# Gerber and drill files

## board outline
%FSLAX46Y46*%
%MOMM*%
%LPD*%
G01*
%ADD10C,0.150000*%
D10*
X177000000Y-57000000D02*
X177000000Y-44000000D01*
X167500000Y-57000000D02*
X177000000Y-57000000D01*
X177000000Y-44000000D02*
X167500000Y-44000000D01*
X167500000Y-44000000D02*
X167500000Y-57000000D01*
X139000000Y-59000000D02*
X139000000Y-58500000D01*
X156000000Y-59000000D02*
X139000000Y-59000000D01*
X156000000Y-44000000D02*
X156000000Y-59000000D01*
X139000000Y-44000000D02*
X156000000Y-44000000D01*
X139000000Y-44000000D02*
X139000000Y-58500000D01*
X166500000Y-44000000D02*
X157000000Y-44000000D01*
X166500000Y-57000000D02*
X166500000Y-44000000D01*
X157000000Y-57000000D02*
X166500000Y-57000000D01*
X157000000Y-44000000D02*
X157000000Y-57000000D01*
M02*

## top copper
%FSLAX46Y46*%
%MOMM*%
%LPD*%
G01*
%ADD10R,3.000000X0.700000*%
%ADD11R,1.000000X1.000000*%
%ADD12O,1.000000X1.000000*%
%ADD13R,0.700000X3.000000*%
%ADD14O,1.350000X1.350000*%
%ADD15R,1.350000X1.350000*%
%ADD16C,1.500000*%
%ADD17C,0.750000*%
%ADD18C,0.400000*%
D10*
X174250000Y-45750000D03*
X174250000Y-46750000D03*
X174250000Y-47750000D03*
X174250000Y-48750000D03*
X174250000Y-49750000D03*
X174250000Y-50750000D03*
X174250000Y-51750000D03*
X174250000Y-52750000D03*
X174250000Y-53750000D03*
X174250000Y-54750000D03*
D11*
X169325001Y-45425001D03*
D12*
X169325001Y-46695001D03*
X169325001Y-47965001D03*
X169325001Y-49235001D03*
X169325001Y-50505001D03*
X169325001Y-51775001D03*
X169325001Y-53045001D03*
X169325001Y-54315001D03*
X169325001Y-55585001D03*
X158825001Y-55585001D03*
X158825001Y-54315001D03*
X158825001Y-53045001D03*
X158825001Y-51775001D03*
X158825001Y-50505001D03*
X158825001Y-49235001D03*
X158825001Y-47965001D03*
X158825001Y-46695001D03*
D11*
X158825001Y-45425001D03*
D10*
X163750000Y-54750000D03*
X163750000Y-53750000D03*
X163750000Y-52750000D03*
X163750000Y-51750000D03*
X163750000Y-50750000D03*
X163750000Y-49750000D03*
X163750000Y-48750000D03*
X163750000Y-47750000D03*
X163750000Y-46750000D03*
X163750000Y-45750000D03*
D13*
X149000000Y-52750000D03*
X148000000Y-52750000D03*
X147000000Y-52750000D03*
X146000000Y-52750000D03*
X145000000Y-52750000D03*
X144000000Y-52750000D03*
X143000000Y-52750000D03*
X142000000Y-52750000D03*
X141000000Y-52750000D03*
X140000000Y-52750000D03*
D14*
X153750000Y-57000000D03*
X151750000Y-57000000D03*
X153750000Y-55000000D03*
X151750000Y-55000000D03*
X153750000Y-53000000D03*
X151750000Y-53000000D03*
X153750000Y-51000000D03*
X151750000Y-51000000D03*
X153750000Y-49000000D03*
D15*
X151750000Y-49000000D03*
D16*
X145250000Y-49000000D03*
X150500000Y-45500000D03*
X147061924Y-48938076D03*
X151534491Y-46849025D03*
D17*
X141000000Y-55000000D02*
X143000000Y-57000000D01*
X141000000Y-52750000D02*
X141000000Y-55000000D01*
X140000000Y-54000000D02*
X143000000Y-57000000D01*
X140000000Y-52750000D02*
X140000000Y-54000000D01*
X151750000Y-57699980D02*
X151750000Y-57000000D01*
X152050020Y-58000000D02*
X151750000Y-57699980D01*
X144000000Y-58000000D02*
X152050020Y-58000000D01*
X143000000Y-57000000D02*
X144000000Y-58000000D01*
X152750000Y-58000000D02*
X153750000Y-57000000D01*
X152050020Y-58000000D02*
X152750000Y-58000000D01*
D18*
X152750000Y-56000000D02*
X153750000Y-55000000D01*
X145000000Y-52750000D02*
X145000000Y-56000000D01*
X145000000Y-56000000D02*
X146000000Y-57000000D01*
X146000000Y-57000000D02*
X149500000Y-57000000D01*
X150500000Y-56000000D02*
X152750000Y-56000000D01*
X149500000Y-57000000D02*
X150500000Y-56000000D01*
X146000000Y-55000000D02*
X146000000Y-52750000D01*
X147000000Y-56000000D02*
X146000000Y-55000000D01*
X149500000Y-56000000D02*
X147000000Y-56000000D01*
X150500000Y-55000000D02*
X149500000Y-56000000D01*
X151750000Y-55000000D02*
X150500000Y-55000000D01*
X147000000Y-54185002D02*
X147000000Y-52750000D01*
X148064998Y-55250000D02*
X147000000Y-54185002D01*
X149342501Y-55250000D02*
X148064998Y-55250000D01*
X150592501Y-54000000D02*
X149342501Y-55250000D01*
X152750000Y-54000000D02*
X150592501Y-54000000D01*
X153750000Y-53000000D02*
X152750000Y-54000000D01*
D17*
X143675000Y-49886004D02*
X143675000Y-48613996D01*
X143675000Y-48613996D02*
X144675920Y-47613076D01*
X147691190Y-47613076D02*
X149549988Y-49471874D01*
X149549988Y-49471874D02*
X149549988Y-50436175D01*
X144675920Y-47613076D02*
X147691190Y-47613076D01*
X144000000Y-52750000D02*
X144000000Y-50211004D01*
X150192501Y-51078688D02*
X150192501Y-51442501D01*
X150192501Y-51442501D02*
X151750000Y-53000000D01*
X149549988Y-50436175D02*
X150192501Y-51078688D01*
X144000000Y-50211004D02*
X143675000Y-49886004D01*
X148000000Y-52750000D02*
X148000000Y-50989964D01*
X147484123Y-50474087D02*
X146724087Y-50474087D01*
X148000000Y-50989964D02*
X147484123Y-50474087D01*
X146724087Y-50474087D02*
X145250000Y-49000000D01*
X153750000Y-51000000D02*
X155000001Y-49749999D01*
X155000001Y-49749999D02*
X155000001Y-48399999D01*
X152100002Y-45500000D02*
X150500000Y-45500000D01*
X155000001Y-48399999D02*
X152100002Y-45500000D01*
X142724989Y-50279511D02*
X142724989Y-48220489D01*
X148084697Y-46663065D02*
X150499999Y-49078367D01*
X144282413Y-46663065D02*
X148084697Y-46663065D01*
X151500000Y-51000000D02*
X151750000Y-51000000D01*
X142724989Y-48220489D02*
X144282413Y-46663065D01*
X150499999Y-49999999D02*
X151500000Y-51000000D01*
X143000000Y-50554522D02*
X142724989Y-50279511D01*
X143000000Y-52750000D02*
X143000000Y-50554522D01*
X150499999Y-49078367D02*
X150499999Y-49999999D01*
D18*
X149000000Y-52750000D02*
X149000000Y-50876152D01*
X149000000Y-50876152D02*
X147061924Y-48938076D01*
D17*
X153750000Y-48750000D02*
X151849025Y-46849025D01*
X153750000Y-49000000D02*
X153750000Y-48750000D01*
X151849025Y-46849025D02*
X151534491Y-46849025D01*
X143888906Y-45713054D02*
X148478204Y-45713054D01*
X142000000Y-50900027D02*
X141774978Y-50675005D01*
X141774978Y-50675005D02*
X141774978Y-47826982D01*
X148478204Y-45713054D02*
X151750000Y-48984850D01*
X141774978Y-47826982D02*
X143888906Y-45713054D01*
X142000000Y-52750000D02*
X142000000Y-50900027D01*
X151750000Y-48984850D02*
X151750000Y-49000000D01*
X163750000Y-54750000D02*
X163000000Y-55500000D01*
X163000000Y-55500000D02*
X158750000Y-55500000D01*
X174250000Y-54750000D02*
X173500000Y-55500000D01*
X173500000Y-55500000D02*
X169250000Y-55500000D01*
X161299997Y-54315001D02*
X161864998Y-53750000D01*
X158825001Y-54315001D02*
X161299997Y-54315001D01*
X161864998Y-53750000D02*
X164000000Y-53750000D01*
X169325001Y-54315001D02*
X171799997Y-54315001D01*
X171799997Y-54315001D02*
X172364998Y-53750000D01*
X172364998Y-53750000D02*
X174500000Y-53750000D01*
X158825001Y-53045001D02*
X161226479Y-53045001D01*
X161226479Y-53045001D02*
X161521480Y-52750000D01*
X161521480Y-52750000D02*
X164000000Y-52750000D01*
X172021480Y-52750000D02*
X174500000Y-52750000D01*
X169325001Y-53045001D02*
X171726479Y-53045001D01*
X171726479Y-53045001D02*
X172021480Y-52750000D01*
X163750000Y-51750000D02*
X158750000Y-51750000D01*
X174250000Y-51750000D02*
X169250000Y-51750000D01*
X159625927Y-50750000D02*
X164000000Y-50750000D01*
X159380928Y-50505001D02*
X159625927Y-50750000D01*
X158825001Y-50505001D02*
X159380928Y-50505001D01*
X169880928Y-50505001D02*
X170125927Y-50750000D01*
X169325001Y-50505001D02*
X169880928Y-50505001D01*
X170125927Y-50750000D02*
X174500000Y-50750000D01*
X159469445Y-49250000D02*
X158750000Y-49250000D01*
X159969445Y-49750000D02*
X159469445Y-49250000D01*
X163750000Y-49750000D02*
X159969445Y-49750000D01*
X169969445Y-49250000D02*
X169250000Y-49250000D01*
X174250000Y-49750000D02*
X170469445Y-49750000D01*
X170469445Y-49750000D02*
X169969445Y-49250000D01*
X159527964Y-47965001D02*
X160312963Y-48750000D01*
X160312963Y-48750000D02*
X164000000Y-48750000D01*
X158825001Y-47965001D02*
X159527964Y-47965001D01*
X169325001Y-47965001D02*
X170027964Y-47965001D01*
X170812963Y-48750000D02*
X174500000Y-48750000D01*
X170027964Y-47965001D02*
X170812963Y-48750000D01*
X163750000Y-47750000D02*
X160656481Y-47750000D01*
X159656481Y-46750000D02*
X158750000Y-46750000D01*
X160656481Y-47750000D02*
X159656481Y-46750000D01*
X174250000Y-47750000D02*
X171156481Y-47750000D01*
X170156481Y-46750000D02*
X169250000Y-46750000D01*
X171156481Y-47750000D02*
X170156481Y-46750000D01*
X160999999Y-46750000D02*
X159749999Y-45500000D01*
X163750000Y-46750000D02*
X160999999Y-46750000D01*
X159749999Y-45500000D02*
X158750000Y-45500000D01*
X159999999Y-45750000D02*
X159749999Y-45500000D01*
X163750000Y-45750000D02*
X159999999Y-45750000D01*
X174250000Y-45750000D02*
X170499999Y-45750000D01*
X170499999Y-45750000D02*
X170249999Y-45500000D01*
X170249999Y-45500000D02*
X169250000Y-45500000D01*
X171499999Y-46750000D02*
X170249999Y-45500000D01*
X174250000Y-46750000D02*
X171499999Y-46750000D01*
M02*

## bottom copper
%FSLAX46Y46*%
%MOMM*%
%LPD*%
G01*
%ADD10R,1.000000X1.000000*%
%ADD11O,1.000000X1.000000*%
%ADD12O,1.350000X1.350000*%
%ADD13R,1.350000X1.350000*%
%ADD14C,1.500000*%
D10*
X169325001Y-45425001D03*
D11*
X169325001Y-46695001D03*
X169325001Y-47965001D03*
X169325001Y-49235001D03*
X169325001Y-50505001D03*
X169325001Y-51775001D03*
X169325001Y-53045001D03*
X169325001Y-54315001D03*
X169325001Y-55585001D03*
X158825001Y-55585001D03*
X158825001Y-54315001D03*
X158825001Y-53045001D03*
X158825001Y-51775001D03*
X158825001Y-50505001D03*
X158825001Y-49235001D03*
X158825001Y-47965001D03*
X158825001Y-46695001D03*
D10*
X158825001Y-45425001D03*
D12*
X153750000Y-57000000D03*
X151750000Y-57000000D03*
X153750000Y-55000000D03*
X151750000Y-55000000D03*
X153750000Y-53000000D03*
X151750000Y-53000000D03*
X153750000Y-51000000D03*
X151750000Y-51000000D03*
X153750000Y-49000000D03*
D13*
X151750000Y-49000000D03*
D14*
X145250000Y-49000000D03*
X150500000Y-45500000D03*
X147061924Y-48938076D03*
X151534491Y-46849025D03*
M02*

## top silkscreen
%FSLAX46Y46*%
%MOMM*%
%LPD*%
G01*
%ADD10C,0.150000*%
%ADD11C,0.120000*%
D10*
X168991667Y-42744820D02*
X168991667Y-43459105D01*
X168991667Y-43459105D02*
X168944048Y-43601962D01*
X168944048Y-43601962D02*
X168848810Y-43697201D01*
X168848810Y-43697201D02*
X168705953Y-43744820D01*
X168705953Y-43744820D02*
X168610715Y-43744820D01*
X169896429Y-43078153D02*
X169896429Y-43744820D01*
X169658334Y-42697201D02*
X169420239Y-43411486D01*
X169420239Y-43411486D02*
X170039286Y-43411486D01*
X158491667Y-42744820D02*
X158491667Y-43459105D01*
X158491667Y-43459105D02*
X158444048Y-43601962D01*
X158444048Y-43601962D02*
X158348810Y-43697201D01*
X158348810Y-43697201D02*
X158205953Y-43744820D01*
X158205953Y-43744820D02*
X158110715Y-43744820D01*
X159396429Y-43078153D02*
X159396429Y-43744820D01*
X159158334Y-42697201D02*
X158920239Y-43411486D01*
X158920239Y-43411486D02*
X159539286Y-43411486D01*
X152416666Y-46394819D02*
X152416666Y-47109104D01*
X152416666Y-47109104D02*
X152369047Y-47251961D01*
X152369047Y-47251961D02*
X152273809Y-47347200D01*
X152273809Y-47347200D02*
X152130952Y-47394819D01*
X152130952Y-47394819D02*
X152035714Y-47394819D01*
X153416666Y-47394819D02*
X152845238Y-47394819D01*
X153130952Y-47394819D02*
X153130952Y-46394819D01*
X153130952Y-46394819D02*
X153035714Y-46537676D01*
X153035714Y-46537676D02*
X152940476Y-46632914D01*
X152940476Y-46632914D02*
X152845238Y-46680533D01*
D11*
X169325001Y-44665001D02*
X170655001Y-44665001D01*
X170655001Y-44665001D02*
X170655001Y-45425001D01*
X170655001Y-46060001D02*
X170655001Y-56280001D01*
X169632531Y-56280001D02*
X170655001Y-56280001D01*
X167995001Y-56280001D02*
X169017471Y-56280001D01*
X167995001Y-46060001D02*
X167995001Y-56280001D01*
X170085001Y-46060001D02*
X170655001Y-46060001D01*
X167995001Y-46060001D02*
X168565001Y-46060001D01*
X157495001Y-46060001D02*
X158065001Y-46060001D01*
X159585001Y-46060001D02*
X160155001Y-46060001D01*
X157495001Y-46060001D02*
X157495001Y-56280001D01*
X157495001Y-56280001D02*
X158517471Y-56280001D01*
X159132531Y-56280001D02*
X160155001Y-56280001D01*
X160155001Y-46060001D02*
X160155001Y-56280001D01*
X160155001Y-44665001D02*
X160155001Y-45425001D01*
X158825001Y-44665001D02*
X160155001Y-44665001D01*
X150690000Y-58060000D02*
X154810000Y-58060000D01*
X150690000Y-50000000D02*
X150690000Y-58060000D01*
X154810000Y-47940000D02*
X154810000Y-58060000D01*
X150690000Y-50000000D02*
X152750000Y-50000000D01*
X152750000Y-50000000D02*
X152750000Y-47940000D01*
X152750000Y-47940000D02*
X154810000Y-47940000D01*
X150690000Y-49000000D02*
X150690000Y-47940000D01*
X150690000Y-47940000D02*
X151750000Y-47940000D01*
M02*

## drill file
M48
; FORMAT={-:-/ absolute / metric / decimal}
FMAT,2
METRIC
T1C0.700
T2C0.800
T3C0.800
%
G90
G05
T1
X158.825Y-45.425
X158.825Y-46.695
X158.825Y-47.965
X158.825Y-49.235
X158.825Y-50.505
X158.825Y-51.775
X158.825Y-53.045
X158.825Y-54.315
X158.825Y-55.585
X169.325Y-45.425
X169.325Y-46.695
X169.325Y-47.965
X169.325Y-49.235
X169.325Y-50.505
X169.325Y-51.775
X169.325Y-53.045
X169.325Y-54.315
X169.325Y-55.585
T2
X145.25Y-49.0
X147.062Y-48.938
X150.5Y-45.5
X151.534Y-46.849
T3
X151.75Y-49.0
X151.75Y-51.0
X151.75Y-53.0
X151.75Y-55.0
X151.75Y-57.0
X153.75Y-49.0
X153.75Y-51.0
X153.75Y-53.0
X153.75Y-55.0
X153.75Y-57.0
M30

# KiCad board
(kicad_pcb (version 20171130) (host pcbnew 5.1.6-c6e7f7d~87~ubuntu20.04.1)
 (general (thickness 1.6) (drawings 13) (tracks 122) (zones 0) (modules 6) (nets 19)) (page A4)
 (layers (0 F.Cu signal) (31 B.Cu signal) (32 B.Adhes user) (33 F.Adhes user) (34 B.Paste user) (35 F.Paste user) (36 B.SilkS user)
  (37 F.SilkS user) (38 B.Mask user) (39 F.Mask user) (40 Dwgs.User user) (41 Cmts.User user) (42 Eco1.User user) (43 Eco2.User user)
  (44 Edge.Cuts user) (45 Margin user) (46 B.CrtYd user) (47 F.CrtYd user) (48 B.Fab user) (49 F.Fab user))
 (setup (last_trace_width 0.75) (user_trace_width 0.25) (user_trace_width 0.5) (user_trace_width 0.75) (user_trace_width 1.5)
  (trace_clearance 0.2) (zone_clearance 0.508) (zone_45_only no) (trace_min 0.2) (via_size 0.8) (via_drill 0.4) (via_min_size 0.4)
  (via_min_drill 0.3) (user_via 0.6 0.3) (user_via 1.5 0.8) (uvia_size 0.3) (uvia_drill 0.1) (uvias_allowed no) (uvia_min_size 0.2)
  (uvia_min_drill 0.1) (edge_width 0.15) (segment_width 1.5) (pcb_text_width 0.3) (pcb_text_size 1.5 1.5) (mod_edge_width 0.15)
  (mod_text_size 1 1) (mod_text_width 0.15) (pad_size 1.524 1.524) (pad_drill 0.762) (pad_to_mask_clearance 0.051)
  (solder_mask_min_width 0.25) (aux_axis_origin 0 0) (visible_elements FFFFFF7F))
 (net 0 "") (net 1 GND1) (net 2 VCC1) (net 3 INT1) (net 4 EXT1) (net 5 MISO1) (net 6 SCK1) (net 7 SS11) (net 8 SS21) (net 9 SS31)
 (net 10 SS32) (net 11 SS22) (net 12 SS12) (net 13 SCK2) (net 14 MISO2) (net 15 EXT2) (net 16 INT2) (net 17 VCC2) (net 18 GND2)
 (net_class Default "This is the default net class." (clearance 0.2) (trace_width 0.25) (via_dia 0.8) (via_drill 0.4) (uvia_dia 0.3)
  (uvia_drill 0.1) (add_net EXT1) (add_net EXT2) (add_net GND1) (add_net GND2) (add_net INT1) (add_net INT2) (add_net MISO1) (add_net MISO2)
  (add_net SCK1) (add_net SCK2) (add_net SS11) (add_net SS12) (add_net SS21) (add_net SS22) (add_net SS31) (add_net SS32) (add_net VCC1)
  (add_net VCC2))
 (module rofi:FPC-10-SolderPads (layer F.Cu) (at 174.25 50.25)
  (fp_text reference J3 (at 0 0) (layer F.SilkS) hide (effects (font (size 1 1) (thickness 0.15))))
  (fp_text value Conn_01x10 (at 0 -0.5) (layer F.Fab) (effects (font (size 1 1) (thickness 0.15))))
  (pad 1 smd rect (at 0 -4.5) (size 3 0.7) (layers F.Cu F.Paste F.Mask) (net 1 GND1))
  (pad 2 smd rect (at 0 -3.5) (size 3 0.7) (layers F.Cu F.Paste F.Mask) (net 1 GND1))
  (pad 3 smd rect (at 0 -2.5) (size 3 0.7) (layers F.Cu F.Paste F.Mask) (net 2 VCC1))
  (pad 4 smd rect (at 0 -1.5) (size 3 0.7) (layers F.Cu F.Paste F.Mask) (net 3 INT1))
  (pad 5 smd rect (at 0 -0.5) (size 3 0.7) (layers F.Cu F.Paste F.Mask) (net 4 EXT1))
  (pad 6 smd rect (at 0 0.5) (size 3 0.7) (layers F.Cu F.Paste F.Mask) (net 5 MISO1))
  (pad 7 smd rect (at 0 1.5) (size 3 0.7) (layers F.Cu F.Paste F.Mask) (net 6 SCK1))
  (pad 8 smd rect (at 0 2.5) (size 3 0.7) (layers F.Cu F.Paste F.Mask) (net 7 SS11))
  (pad 9 smd rect (at 0 3.5) (size 3 0.7) (layers F.Cu F.Paste F.Mask) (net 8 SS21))
  (pad 10 smd rect (at 0 4.5) (size 3 0.7) (layers F.Cu F.Paste F.Mask) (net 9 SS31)))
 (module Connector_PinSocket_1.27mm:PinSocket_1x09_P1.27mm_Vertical (layer F.Cu) (at 169.325001 45.425001)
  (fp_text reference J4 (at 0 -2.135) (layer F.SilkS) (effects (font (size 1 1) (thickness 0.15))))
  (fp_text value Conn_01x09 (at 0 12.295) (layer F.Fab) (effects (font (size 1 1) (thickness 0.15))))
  (fp_line (start 0 -0.76) (end 1.33 -0.76) (layer F.SilkS) (width 0.12))
  (fp_line (start 1.33 -0.76) (end 1.33 0) (layer F.SilkS) (width 0.12))
  (fp_line (start 1.33 0.635) (end 1.33 10.855) (layer F.SilkS) (width 0.12))
  (fp_line (start 0.30753 10.855) (end 1.33 10.855) (layer F.SilkS) (width 0.12))
  (fp_line (start -1.33 10.855) (end -0.30753 10.855) (layer F.SilkS) (width 0.12))
  (fp_line (start -1.33 0.635) (end -1.33 10.855) (layer F.SilkS) (width 0.12))
  (fp_line (start 0.76 0.635) (end 1.33 0.635) (layer F.SilkS) (width 0.12))
  (fp_line (start -1.33 0.635) (end -0.76 0.635) (layer F.SilkS) (width 0.12))
  (pad 1 thru_hole rect (at 0 0) (size 1 1) (drill 0.7) (layers *.Cu *.Mask) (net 1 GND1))
  (pad 2 thru_hole oval (at 0 1.27) (size 1 1) (drill 0.7) (layers *.Cu *.Mask) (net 2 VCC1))
  (pad 3 thru_hole oval (at 0 2.54) (size 1 1) (drill 0.7) (layers *.Cu *.Mask) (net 3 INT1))
  (pad 4 thru_hole oval (at 0 3.81) (size 1 1) (drill 0.7) (layers *.Cu *.Mask) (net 4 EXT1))
  (pad 5 thru_hole oval (at 0 5.08) (size 1 1) (drill 0.7) (layers *.Cu *.Mask) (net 5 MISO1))
  (pad 6 thru_hole oval (at 0 6.35) (size 1 1) (drill 0.7) (layers *.Cu *.Mask) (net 6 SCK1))
  (pad 7 thru_hole oval (at 0 7.62) (size 1 1) (drill 0.7) (layers *.Cu *.Mask) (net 7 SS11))
  (pad 8 thru_hole oval (at 0 8.89) (size 1 1) (drill 0.7) (layers *.Cu *.Mask) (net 8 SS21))
  (pad 9 thru_hole oval (at 0 10.16) (size 1 1) (drill 0.7) (layers *.Cu *.Mask) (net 9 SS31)))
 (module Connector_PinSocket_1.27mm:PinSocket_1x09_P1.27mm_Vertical (layer F.Cu) (at 158.825001 45.425001)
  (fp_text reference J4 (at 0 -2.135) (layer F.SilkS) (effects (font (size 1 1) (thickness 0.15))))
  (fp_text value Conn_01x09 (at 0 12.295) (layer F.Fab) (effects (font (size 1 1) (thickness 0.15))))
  (fp_line (start -1.33 0.635) (end -0.76 0.635) (layer F.SilkS) (width 0.12))
  (fp_line (start 0.76 0.635) (end 1.33 0.635) (layer F.SilkS) (width 0.12))
  (fp_line (start -1.33 0.635) (end -1.33 10.855) (layer F.SilkS) (width 0.12))
  (fp_line (start -1.33 10.855) (end -0.30753 10.855) (layer F.SilkS) (width 0.12))
  (fp_line (start 0.30753 10.855) (end 1.33 10.855) (layer F.SilkS) (width 0.12))
  (fp_line (start 1.33 0.635) (end 1.33 10.855) (layer F.SilkS) (width 0.12))
  (fp_line (start 1.33 -0.76) (end 1.33 0) (layer F.SilkS) (width 0.12))
  (fp_line (start 0 -0.76) (end 1.33 -0.76) (layer F.SilkS) (width 0.12))
  (pad 9 thru_hole oval (at 0 10.16) (size 1 1) (drill 0.7) (layers *.Cu *.Mask) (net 9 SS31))
  (pad 8 thru_hole oval (at 0 8.89) (size 1 1) (drill 0.7) (layers *.Cu *.Mask) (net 8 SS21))
  (pad 7 thru_hole oval (at 0 7.62) (size 1 1) (drill 0.7) (layers *.Cu *.Mask) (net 7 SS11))
  (pad 6 thru_hole oval (at 0 6.35) (size 1 1) (drill 0.7) (layers *.Cu *.Mask) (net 6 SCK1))
  (pad 5 thru_hole oval (at 0 5.08) (size 1 1) (drill 0.7) (layers *.Cu *.Mask) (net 5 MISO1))
  (pad 4 thru_hole oval (at 0 3.81) (size 1 1) (drill 0.7) (layers *.Cu *.Mask) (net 4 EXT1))
  (pad 3 thru_hole oval (at 0 2.54) (size 1 1) (drill 0.7) (layers *.Cu *.Mask) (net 3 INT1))
  (pad 2 thru_hole oval (at 0 1.27) (size 1 1) (drill 0.7) (layers *.Cu *.Mask) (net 2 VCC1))
  (pad 1 thru_hole rect (at 0 0) (size 1 1) (drill 0.7) (layers *.Cu *.Mask) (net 1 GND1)))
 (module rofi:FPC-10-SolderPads (layer F.Cu) (at 163.75 50.25)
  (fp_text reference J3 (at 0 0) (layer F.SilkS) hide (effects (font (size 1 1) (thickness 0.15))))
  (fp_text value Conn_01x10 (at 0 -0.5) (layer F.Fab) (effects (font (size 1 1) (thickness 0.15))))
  (pad 10 smd rect (at 0 4.5) (size 3 0.7) (layers F.Cu F.Paste F.Mask) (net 9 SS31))
  (pad 9 smd rect (at 0 3.5) (size 3 0.7) (layers F.Cu F.Paste F.Mask) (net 8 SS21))
  (pad 8 smd rect (at 0 2.5) (size 3 0.7) (layers F.Cu F.Paste F.Mask) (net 7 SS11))
  (pad 7 smd rect (at 0 1.5) (size 3 0.7) (layers F.Cu F.Paste F.Mask) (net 6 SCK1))
  (pad 6 smd rect (at 0 0.5) (size 3 0.7) (layers F.Cu F.Paste F.Mask) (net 5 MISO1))
  (pad 5 smd rect (at 0 -0.5) (size 3 0.7) (layers F.Cu F.Paste F.Mask) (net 4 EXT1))
  (pad 4 smd rect (at 0 -1.5) (size 3 0.7) (layers F.Cu F.Paste F.Mask) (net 3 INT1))
  (pad 3 smd rect (at 0 -2.5) (size 3 0.7) (layers F.Cu F.Paste F.Mask) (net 2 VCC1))
  (pad 2 smd rect (at 0 -3.5) (size 3 0.7) (layers F.Cu F.Paste F.Mask) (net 1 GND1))
  (pad 1 smd rect (at 0 -4.5) (size 3 0.7) (layers F.Cu F.Paste F.Mask) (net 1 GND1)))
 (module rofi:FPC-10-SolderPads (layer F.Cu) (at 144.5 52.75 90)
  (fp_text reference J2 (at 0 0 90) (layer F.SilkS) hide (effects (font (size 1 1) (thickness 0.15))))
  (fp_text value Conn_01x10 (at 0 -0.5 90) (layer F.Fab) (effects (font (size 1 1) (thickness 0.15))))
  (pad 10 smd rect (at 0 4.5 90) (size 3 0.7) (layers F.Cu F.Paste F.Mask) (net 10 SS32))
  (pad 9 smd rect (at 0 3.5 90) (size 3 0.7) (layers F.Cu F.Paste F.Mask) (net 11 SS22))
  (pad 8 smd rect (at 0 2.5 90) (size 3 0.7) (layers F.Cu F.Paste F.Mask) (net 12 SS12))
  (pad 7 smd rect (at 0 1.5 90) (size 3 0.7) (layers F.Cu F.Paste F.Mask) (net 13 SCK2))
  (pad 6 smd rect (at 0 0.5 90) (size 3 0.7) (layers F.Cu F.Paste F.Mask) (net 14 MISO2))
  (pad 5 smd rect (at 0 -0.5 90) (size 3 0.7) (layers F.Cu F.Paste F.Mask) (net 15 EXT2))
  (pad 4 smd rect (at 0 -1.5 90) (size 3 0.7) (layers F.Cu F.Paste F.Mask) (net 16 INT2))
  (pad 3 smd rect (at 0 -2.5 90) (size 3 0.7) (layers F.Cu F.Paste F.Mask) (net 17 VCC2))
  (pad 2 smd rect (at 0 -3.5 90) (size 3 0.7) (layers F.Cu F.Paste F.Mask) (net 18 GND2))
  (pad 1 smd rect (at 0 -4.5 90) (size 3 0.7) (layers F.Cu F.Paste F.Mask) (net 18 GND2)))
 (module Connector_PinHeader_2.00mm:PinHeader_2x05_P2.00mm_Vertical (layer F.Cu) (at 151.75 49)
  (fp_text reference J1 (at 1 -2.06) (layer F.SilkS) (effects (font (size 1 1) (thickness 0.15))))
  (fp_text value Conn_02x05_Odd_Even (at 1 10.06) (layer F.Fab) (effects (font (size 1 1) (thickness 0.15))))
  (fp_line (start -1.06 9.06) (end 3.06 9.06) (layer F.SilkS) (width 0.12))
  (fp_line (start -1.06 1) (end -1.06 9.06) (layer F.SilkS) (width 0.12))
  (fp_line (start 3.06 -1.06) (end 3.06 9.06) (layer F.SilkS) (width 0.12))
  (fp_line (start -1.06 1) (end 1 1) (layer F.SilkS) (width 0.12))
  (fp_line (start 1 1) (end 1 -1.06) (layer F.SilkS) (width 0.12))
  (fp_line (start 1 -1.06) (end 3.06 -1.06) (layer F.SilkS) (width 0.12))
  (fp_line (start -1.06 0) (end -1.06 -1.06) (layer F.SilkS) (width 0.12))
  (fp_line (start -1.06 -1.06) (end 0 -1.06) (layer F.SilkS) (width 0.12))
  (pad 10 thru_hole oval (at 2 8) (size 1.35 1.35) (drill 0.8) (layers *.Cu *.Mask) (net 18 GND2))
  (pad 9 thru_hole oval (at 0 8) (size 1.35 1.35) (drill 0.8) (layers *.Cu *.Mask) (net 18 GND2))
  (pad 8 thru_hole oval (at 2 6) (size 1.35 1.35) (drill 0.8) (layers *.Cu *.Mask) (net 14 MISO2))
  (pad 7 thru_hole oval (at 0 6) (size 1.35 1.35) (drill 0.8) (layers *.Cu *.Mask) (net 13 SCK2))
  (pad 6 thru_hole oval (at 2 4) (size 1.35 1.35) (drill 0.8) (layers *.Cu *.Mask) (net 12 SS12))
  (pad 5 thru_hole oval (at 0 4) (size 1.35 1.35) (drill 0.8) (layers *.Cu *.Mask) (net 15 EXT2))
  (pad 4 thru_hole oval (at 2 2) (size 1.35 1.35) (drill 0.8) (layers *.Cu *.Mask) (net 11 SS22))
  (pad 3 thru_hole oval (at 0 2) (size 1.35 1.35) (drill 0.8) (layers *.Cu *.Mask) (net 16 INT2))
  (pad 2 thru_hole oval (at 2 0) (size 1.35 1.35) (drill 0.8) (layers *.Cu *.Mask) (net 10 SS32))
  (pad 1 thru_hole rect (at 0 0) (size 1.35 1.35) (drill 0.8) (layers *.Cu *.Mask) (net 17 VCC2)))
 (gr_line (start 177 57) (end 177 44) (layer Edge.Cuts) (width 0.15))
 (gr_line (start 167.5 57) (end 177 57) (layer Edge.Cuts) (width 0.15))
 (gr_line (start 177 44) (end 167.5 44) (layer Edge.Cuts) (width 0.15))
 (gr_line (start 167.5 44) (end 167.5 57) (layer Edge.Cuts) (width 0.15))
 (gr_line (start 139 59) (end 139 58.5) (layer Edge.Cuts) (width 0.15))
 (gr_line (start 156 59) (end 139 59) (layer Edge.Cuts) (width 0.15))
 (gr_line (start 156 44) (end 156 59) (layer Edge.Cuts) (width 0.15))
 (gr_line (start 139 44) (end 156 44) (layer Edge.Cuts) (width 0.15))
 (gr_line (start 139 44) (end 139 58.5) (layer Edge.Cuts) (width 0.15))
 (gr_line (start 166.5 44) (end 157 44) (layer Edge.Cuts) (width 0.15))
 (gr_line (start 166.5 57) (end 166.5 44) (layer Edge.Cuts) (width 0.15))
 (gr_line (start 157 57) (end 166.5 57) (layer Edge.Cuts) (width 0.15))
 (gr_line (start 157 44) (end 157 57) (layer Edge.Cuts) (width 0.15))
 (segment (start 141 55) (end 143 57) (width 0.75) (layer F.Cu) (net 18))
 (segment (start 141 52.75) (end 141 55) (width 0.75) (layer F.Cu) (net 18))
 (segment (start 140 54) (end 143 57) (width 0.75) (layer F.Cu) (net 18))
 (segment (start 140 52.75) (end 140 54) (width 0.75) (layer F.Cu) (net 18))
 (segment (start 151.75 57.69998) (end 151.75 57) (width 0.75) (layer F.Cu) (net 18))
 (segment (start 152.05002 58) (end 151.75 57.69998) (width 0.75) (layer F.Cu) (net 18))
 (segment (start 144 58) (end 152.05002 58) (width 0.75) (layer F.Cu) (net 18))
 (segment (start 143 57) (end 144 58) (width 0.75) (layer F.Cu) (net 18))
 (segment (start 152.75 58) (end 153.75 57) (width 0.75) (layer F.Cu) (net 18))
 (segment (start 152.05002 58) (end 152.75 58) (width 0.75) (layer F.Cu) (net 18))
 (segment (start 152.75 56) (end 153.75 55) (width 0.4) (layer F.Cu) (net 14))
 (segment (start 145 52.75) (end 145 56) (width 0.4) (layer F.Cu) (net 14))
 (segment (start 145 56) (end 146 57) (width 0.4) (layer F.Cu) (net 14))
 (segment (start 146 57) (end 149.5 57) (width 0.4) (layer F.Cu) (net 14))
 (segment (start 150.5 56) (end 152.75 56) (width 0.4) (layer F.Cu) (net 14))
 (segment (start 149.5 57) (end 150.5 56) (width 0.4) (layer F.Cu) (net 14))
 (segment (start 146 55) (end 146 52.75) (width 0.4) (layer F.Cu) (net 13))
 (segment (start 147 56) (end 146 55) (width 0.4) (layer F.Cu) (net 13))
 (segment (start 149.5 56) (end 147 56) (width 0.4) (layer F.Cu) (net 13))
 (segment (start 150.5 55) (end 149.5 56) (width 0.4) (layer F.Cu) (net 13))
 (segment (start 151.75 55) (end 150.5 55) (width 0.4) (layer F.Cu) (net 13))
 (segment (start 147 54.185002) (end 147 52.75) (width 0.4) (layer F.Cu) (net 12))
 (segment (start 148.064998 55.25) (end 147 54.185002) (width 0.4) (layer F.Cu) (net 12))
 (segment (start 149.342501 55.25) (end 148.064998 55.25) (width 0.4) (layer F.Cu) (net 12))
 (segment (start 150.592501 54) (end 149.342501 55.25) (width 0.4) (layer F.Cu) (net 12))
 (segment (start 152.75 54) (end 150.592501 54) (width 0.4) (layer F.Cu) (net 12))
 (segment (start 153.75 53) (end 152.75 54) (width 0.4) (layer F.Cu) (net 12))
 (segment (start 143.675 49.886004) (end 143.675 48.613996) (width 0.75) (layer F.Cu) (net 15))
 (segment (start 143.675 48.613996) (end 144.67592 47.613076) (width 0.75) (layer F.Cu) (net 15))
 (segment (start 147.69119 47.613076) (end 149.549988 49.471874) (width 0.75) (layer F.Cu) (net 15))
 (segment (start 149.549988 49.471874) (end 149.549988 50.436175) (width 0.75) (layer F.Cu) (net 15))
 (segment (start 144.67592 47.613076) (end 147.69119 47.613076) (width 0.75) (layer F.Cu) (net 15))
 (segment (start 144 52.75) (end 144 50.211004) (width 0.75) (layer F.Cu) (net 15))
 (segment (start 150.192501 51.078688) (end 150.192501 51.442501) (width 0.75) (layer F.Cu) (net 15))
 (segment (start 150.192501 51.442501) (end 151.75 53) (width 0.75) (layer F.Cu) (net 15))
 (segment (start 149.549988 50.436175) (end 150.192501 51.078688) (width 0.75) (layer F.Cu) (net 15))
 (segment (start 144 50.211004) (end 143.675 49.886004) (width 0.75) (layer F.Cu) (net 15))
 (segment (start 148 52.75) (end 148 50.989964) (width 0.75) (layer F.Cu) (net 11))
 (via (at 145.25 49) (size 1.5) (drill 0.8) (layers F.Cu B.Cu) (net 11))
 (segment (start 147.484123 50.474087) (end 146.724087 50.474087) (width 0.75) (layer F.Cu) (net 11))
 (segment (start 148 50.989964) (end 147.484123 50.474087) (width 0.75) (layer F.Cu) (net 11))
 (segment (start 146.724087 50.474087) (end 145.25 49) (width 0.75) (layer F.Cu) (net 11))
 (segment (start 153.75 51) (end 155.000001 49.749999) (width 0.75) (layer F.Cu) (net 11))
 (segment (start 155.000001 49.749999) (end 155.000001 48.399999) (width 0.75) (layer F.Cu) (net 11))
 (segment (start 152.100002 45.5) (end 150.5 45.5) (width 0.75) (layer F.Cu) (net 11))
 (segment (start 155.000001 48.399999) (end 152.100002 45.5) (width 0.75) (layer F.Cu) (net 11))
 (via (at 150.5 45.5) (size 1.5) (drill 0.8) (layers F.Cu B.Cu) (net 11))
 (segment (start 142.724989 50.279511) (end 142.724989 48.220489) (width 0.75) (layer F.Cu) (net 16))
 (segment (start 148.084697 46.663065) (end 150.499999 49.078367) (width 0.75) (layer F.Cu) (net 16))
 (segment (start 144.282413 46.663065) (end 148.084697 46.663065) (width 0.75) (layer F.Cu) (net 16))
 (segment (start 151.5 51) (end 151.75 51) (width 0.75) (layer F.Cu) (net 16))
 (segment (start 142.724989 48.220489) (end 144.282413 46.663065) (width 0.75) (layer F.Cu) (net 16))
 (segment (start 150.499999 49.999999) (end 151.5 51) (width 0.75) (layer F.Cu) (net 16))
 (segment (start 143 50.554522) (end 142.724989 50.279511) (width 0.75) (layer F.Cu) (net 16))
 (segment (start 143 52.75) (end 143 50.554522) (width 0.75) (layer F.Cu) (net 16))
 (segment (start 150.499999 49.078367) (end 150.499999 49.999999) (width 0.75) (layer F.Cu) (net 16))
 (segment (start 149 52.75) (end 149 50.876152) (width 0.4) (layer F.Cu) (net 10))
 (segment (start 149 50.876152) (end 147.061924 48.938076) (width 0.4) (layer F.Cu) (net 10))
 (via (at 147.061924 48.938076) (size 1.5) (drill 0.8) (layers F.Cu B.Cu) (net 10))
 (segment (start 153.75 48.75) (end 151.849025 46.849025) (width 0.75) (layer F.Cu) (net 10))
 (segment (start 153.75 49) (end 153.75 48.75) (width 0.75) (layer F.Cu) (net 10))
 (segment (start 151.849025 46.849025) (end 151.534491 46.849025) (width 0.75) (layer F.Cu) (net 10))
 (via (at 151.534491 46.849025) (size 1.5) (drill 0.8) (layers F.Cu B.Cu) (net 10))
 (segment (start 143.888906 45.713054) (end 148.478204 45.713054) (width 0.75) (layer F.Cu) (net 17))
 (segment (start 142 50.900027) (end 141.774978 50.675005) (width 0.75) (layer F.Cu) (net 17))
 (segment (start 141.774978 50.675005) (end 141.774978 47.826982) (width 0.75) (layer F.Cu) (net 17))
 (segment (start 148.478204 45.713054) (end 151.75 48.98485) (width 0.75) (layer F.Cu) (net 17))
 (segment (start 141.774978 47.826982) (end 143.888906 45.713054) (width 0.75) (layer F.Cu) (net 17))
 (segment (start 142 52.75) (end 142 50.900027) (width 0.75) (layer F.Cu) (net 17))
 (segment (start 151.75 48.98485) (end 151.75 49) (width 0.75) (layer F.Cu) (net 17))
 (segment (start 163.75 54.75) (end 163 55.5) (width 0.75) (layer F.Cu) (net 9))
 (segment (start 163 55.5) (end 158.75 55.5) (width 0.75) (layer F.Cu) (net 9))
 (segment (start 174.25 54.75) (end 173.5 55.5) (width 0.75) (layer F.Cu) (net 9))
 (segment (start 173.5 55.5) (end 169.25 55.5) (width 0.75) (layer F.Cu) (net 9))
 (segment (start 161.299997 54.315001) (end 161.864998 53.75) (width 0.75) (layer F.Cu) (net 8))
 (segment (start 158.825001 54.315001) (end 161.299997 54.315001) (width 0.75) (layer F.Cu) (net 8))
 (segment (start 161.864998 53.75) (end 164 53.75) (width 0.75) (layer F.Cu) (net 8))
 (segment (start 169.325001 54.315001) (end 171.799997 54.315001) (width 0.75) (layer F.Cu) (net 8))
 (segment (start 171.799997 54.315001) (end 172.364998 53.75) (width 0.75) (layer F.Cu) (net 8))
 (segment (start 172.364998 53.75) (end 174.5 53.75) (width 0.75) (layer F.Cu) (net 8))
 (segment (start 158.825001 53.045001) (end 161.226479 53.045001) (width 0.75) (layer F.Cu) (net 7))
 (segment (start 161.226479 53.045001) (end 161.52148 52.75) (width 0.75) (layer F.Cu) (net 7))
 (segment (start 161.52148 52.75) (end 164 52.75) (width 0.75) (layer F.Cu) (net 7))
 (segment (start 172.02148 52.75) (end 174.5 52.75) (width 0.75) (layer F.Cu) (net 7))
 (segment (start 169.325001 53.045001) (end 171.726479 53.045001) (width 0.75) (layer F.Cu) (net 7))
 (segment (start 171.726479 53.045001) (end 172.02148 52.75) (width 0.75) (layer F.Cu) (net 7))
 (segment (start 163.75 51.75) (end 158.75 51.75) (width 0.75) (layer F.Cu) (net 6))
 (segment (start 174.25 51.75) (end 169.25 51.75) (width 0.75) (layer F.Cu) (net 6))
 (segment (start 159.625927 50.75) (end 164 50.75) (width 0.75) (layer F.Cu) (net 5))
 (segment (start 159.380928 50.505001) (end 159.625927 50.75) (width 0.75) (layer F.Cu) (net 5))
 (segment (start 158.825001 50.505001) (end 159.380928 50.505001) (width 0.75) (layer F.Cu) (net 5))
 (segment (start 169.880928 50.505001) (end 170.125927 50.75) (width 0.75) (layer F.Cu) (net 5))
 (segment (start 169.325001 50.505001) (end 169.880928 50.505001) (width 0.75) (layer F.Cu) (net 5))
 (segment (start 170.125927 50.75) (end 174.5 50.75) (width 0.75) (layer F.Cu) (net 5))
 (segment (start 159.469445 49.25) (end 158.75 49.25) (width 0.75) (layer F.Cu) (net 4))
 (segment (start 159.969445 49.75) (end 159.469445 49.25) (width 0.75) (layer F.Cu) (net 4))
 (segment (start 163.75 49.75) (end 159.969445 49.75) (width 0.75) (layer F.Cu) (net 4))
 (segment (start 169.969445 49.25) (end 169.25 49.25) (width 0.75) (layer F.Cu) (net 4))
 (segment (start 174.25 49.75) (end 170.469445 49.75) (width 0.75) (layer F.Cu) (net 4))
 (segment (start 170.469445 49.75) (end 169.969445 49.25) (width 0.75) (layer F.Cu) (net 4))
 (segment (start 159.527964 47.965001) (end 160.312963 48.75) (width 0.75) (layer F.Cu) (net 3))
 (segment (start 160.312963 48.75) (end 164 48.75) (width 0.75) (layer F.Cu) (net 3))
 (segment (start 158.825001 47.965001) (end 159.527964 47.965001) (width 0.75) (layer F.Cu) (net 3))
 (segment (start 169.325001 47.965001) (end 170.027964 47.965001) (width 0.75) (layer F.Cu) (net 3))
 (segment (start 170.812963 48.75) (end 174.5 48.75) (width 0.75) (layer F.Cu) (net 3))
 (segment (start 170.027964 47.965001) (end 170.812963 48.75) (width 0.75) (layer F.Cu) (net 3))
 (segment (start 163.75 47.75) (end 160.656481 47.75) (width 0.75) (layer F.Cu) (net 2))
 (segment (start 159.656481 46.75) (end 158.75 46.75) (width 0.75) (layer F.Cu) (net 2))
 (segment (start 160.656481 47.75) (end 159.656481 46.75) (width 0.75) (layer F.Cu) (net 2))
 (segment (start 174.25 47.75) (end 171.156481 47.75) (width 0.75) (layer F.Cu) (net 2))
 (segment (start 170.156481 46.75) (end 169.25 46.75) (width 0.75) (layer F.Cu) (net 2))
 (segment (start 171.156481 47.75) (end 170.156481 46.75) (width 0.75) (layer F.Cu) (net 2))
 (segment (start 160.999999 46.75) (end 159.749999 45.5) (width 0.75) (layer F.Cu) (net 1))
 (segment (start 163.75 46.75) (end 160.999999 46.75) (width 0.75) (layer F.Cu) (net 1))
 (segment (start 159.749999 45.5) (end 158.75 45.5) (width 0.75) (layer F.Cu) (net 1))
 (segment (start 159.999999 45.75) (end 159.749999 45.5) (width 0.75) (layer F.Cu) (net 1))
 (segment (start 163.75 45.75) (end 159.999999 45.75) (width 0.75) (layer F.Cu) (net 1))
 (segment (start 174.25 45.75) (end 170.499999 45.75) (width 0.75) (layer F.Cu) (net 1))
 (segment (start 170.499999 45.75) (end 170.249999 45.5) (width 0.75) (layer F.Cu) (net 1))
 (segment (start 170.249999 45.5) (end 169.25 45.5) (width 0.75) (layer F.Cu) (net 1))
 (segment (start 171.499999 46.75) (end 170.249999 45.5) (width 0.75) (layer F.Cu) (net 1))
 (segment (start 174.25 46.75) (end 171.499999 46.75) (width 0.75) (layer F.Cu) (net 1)))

